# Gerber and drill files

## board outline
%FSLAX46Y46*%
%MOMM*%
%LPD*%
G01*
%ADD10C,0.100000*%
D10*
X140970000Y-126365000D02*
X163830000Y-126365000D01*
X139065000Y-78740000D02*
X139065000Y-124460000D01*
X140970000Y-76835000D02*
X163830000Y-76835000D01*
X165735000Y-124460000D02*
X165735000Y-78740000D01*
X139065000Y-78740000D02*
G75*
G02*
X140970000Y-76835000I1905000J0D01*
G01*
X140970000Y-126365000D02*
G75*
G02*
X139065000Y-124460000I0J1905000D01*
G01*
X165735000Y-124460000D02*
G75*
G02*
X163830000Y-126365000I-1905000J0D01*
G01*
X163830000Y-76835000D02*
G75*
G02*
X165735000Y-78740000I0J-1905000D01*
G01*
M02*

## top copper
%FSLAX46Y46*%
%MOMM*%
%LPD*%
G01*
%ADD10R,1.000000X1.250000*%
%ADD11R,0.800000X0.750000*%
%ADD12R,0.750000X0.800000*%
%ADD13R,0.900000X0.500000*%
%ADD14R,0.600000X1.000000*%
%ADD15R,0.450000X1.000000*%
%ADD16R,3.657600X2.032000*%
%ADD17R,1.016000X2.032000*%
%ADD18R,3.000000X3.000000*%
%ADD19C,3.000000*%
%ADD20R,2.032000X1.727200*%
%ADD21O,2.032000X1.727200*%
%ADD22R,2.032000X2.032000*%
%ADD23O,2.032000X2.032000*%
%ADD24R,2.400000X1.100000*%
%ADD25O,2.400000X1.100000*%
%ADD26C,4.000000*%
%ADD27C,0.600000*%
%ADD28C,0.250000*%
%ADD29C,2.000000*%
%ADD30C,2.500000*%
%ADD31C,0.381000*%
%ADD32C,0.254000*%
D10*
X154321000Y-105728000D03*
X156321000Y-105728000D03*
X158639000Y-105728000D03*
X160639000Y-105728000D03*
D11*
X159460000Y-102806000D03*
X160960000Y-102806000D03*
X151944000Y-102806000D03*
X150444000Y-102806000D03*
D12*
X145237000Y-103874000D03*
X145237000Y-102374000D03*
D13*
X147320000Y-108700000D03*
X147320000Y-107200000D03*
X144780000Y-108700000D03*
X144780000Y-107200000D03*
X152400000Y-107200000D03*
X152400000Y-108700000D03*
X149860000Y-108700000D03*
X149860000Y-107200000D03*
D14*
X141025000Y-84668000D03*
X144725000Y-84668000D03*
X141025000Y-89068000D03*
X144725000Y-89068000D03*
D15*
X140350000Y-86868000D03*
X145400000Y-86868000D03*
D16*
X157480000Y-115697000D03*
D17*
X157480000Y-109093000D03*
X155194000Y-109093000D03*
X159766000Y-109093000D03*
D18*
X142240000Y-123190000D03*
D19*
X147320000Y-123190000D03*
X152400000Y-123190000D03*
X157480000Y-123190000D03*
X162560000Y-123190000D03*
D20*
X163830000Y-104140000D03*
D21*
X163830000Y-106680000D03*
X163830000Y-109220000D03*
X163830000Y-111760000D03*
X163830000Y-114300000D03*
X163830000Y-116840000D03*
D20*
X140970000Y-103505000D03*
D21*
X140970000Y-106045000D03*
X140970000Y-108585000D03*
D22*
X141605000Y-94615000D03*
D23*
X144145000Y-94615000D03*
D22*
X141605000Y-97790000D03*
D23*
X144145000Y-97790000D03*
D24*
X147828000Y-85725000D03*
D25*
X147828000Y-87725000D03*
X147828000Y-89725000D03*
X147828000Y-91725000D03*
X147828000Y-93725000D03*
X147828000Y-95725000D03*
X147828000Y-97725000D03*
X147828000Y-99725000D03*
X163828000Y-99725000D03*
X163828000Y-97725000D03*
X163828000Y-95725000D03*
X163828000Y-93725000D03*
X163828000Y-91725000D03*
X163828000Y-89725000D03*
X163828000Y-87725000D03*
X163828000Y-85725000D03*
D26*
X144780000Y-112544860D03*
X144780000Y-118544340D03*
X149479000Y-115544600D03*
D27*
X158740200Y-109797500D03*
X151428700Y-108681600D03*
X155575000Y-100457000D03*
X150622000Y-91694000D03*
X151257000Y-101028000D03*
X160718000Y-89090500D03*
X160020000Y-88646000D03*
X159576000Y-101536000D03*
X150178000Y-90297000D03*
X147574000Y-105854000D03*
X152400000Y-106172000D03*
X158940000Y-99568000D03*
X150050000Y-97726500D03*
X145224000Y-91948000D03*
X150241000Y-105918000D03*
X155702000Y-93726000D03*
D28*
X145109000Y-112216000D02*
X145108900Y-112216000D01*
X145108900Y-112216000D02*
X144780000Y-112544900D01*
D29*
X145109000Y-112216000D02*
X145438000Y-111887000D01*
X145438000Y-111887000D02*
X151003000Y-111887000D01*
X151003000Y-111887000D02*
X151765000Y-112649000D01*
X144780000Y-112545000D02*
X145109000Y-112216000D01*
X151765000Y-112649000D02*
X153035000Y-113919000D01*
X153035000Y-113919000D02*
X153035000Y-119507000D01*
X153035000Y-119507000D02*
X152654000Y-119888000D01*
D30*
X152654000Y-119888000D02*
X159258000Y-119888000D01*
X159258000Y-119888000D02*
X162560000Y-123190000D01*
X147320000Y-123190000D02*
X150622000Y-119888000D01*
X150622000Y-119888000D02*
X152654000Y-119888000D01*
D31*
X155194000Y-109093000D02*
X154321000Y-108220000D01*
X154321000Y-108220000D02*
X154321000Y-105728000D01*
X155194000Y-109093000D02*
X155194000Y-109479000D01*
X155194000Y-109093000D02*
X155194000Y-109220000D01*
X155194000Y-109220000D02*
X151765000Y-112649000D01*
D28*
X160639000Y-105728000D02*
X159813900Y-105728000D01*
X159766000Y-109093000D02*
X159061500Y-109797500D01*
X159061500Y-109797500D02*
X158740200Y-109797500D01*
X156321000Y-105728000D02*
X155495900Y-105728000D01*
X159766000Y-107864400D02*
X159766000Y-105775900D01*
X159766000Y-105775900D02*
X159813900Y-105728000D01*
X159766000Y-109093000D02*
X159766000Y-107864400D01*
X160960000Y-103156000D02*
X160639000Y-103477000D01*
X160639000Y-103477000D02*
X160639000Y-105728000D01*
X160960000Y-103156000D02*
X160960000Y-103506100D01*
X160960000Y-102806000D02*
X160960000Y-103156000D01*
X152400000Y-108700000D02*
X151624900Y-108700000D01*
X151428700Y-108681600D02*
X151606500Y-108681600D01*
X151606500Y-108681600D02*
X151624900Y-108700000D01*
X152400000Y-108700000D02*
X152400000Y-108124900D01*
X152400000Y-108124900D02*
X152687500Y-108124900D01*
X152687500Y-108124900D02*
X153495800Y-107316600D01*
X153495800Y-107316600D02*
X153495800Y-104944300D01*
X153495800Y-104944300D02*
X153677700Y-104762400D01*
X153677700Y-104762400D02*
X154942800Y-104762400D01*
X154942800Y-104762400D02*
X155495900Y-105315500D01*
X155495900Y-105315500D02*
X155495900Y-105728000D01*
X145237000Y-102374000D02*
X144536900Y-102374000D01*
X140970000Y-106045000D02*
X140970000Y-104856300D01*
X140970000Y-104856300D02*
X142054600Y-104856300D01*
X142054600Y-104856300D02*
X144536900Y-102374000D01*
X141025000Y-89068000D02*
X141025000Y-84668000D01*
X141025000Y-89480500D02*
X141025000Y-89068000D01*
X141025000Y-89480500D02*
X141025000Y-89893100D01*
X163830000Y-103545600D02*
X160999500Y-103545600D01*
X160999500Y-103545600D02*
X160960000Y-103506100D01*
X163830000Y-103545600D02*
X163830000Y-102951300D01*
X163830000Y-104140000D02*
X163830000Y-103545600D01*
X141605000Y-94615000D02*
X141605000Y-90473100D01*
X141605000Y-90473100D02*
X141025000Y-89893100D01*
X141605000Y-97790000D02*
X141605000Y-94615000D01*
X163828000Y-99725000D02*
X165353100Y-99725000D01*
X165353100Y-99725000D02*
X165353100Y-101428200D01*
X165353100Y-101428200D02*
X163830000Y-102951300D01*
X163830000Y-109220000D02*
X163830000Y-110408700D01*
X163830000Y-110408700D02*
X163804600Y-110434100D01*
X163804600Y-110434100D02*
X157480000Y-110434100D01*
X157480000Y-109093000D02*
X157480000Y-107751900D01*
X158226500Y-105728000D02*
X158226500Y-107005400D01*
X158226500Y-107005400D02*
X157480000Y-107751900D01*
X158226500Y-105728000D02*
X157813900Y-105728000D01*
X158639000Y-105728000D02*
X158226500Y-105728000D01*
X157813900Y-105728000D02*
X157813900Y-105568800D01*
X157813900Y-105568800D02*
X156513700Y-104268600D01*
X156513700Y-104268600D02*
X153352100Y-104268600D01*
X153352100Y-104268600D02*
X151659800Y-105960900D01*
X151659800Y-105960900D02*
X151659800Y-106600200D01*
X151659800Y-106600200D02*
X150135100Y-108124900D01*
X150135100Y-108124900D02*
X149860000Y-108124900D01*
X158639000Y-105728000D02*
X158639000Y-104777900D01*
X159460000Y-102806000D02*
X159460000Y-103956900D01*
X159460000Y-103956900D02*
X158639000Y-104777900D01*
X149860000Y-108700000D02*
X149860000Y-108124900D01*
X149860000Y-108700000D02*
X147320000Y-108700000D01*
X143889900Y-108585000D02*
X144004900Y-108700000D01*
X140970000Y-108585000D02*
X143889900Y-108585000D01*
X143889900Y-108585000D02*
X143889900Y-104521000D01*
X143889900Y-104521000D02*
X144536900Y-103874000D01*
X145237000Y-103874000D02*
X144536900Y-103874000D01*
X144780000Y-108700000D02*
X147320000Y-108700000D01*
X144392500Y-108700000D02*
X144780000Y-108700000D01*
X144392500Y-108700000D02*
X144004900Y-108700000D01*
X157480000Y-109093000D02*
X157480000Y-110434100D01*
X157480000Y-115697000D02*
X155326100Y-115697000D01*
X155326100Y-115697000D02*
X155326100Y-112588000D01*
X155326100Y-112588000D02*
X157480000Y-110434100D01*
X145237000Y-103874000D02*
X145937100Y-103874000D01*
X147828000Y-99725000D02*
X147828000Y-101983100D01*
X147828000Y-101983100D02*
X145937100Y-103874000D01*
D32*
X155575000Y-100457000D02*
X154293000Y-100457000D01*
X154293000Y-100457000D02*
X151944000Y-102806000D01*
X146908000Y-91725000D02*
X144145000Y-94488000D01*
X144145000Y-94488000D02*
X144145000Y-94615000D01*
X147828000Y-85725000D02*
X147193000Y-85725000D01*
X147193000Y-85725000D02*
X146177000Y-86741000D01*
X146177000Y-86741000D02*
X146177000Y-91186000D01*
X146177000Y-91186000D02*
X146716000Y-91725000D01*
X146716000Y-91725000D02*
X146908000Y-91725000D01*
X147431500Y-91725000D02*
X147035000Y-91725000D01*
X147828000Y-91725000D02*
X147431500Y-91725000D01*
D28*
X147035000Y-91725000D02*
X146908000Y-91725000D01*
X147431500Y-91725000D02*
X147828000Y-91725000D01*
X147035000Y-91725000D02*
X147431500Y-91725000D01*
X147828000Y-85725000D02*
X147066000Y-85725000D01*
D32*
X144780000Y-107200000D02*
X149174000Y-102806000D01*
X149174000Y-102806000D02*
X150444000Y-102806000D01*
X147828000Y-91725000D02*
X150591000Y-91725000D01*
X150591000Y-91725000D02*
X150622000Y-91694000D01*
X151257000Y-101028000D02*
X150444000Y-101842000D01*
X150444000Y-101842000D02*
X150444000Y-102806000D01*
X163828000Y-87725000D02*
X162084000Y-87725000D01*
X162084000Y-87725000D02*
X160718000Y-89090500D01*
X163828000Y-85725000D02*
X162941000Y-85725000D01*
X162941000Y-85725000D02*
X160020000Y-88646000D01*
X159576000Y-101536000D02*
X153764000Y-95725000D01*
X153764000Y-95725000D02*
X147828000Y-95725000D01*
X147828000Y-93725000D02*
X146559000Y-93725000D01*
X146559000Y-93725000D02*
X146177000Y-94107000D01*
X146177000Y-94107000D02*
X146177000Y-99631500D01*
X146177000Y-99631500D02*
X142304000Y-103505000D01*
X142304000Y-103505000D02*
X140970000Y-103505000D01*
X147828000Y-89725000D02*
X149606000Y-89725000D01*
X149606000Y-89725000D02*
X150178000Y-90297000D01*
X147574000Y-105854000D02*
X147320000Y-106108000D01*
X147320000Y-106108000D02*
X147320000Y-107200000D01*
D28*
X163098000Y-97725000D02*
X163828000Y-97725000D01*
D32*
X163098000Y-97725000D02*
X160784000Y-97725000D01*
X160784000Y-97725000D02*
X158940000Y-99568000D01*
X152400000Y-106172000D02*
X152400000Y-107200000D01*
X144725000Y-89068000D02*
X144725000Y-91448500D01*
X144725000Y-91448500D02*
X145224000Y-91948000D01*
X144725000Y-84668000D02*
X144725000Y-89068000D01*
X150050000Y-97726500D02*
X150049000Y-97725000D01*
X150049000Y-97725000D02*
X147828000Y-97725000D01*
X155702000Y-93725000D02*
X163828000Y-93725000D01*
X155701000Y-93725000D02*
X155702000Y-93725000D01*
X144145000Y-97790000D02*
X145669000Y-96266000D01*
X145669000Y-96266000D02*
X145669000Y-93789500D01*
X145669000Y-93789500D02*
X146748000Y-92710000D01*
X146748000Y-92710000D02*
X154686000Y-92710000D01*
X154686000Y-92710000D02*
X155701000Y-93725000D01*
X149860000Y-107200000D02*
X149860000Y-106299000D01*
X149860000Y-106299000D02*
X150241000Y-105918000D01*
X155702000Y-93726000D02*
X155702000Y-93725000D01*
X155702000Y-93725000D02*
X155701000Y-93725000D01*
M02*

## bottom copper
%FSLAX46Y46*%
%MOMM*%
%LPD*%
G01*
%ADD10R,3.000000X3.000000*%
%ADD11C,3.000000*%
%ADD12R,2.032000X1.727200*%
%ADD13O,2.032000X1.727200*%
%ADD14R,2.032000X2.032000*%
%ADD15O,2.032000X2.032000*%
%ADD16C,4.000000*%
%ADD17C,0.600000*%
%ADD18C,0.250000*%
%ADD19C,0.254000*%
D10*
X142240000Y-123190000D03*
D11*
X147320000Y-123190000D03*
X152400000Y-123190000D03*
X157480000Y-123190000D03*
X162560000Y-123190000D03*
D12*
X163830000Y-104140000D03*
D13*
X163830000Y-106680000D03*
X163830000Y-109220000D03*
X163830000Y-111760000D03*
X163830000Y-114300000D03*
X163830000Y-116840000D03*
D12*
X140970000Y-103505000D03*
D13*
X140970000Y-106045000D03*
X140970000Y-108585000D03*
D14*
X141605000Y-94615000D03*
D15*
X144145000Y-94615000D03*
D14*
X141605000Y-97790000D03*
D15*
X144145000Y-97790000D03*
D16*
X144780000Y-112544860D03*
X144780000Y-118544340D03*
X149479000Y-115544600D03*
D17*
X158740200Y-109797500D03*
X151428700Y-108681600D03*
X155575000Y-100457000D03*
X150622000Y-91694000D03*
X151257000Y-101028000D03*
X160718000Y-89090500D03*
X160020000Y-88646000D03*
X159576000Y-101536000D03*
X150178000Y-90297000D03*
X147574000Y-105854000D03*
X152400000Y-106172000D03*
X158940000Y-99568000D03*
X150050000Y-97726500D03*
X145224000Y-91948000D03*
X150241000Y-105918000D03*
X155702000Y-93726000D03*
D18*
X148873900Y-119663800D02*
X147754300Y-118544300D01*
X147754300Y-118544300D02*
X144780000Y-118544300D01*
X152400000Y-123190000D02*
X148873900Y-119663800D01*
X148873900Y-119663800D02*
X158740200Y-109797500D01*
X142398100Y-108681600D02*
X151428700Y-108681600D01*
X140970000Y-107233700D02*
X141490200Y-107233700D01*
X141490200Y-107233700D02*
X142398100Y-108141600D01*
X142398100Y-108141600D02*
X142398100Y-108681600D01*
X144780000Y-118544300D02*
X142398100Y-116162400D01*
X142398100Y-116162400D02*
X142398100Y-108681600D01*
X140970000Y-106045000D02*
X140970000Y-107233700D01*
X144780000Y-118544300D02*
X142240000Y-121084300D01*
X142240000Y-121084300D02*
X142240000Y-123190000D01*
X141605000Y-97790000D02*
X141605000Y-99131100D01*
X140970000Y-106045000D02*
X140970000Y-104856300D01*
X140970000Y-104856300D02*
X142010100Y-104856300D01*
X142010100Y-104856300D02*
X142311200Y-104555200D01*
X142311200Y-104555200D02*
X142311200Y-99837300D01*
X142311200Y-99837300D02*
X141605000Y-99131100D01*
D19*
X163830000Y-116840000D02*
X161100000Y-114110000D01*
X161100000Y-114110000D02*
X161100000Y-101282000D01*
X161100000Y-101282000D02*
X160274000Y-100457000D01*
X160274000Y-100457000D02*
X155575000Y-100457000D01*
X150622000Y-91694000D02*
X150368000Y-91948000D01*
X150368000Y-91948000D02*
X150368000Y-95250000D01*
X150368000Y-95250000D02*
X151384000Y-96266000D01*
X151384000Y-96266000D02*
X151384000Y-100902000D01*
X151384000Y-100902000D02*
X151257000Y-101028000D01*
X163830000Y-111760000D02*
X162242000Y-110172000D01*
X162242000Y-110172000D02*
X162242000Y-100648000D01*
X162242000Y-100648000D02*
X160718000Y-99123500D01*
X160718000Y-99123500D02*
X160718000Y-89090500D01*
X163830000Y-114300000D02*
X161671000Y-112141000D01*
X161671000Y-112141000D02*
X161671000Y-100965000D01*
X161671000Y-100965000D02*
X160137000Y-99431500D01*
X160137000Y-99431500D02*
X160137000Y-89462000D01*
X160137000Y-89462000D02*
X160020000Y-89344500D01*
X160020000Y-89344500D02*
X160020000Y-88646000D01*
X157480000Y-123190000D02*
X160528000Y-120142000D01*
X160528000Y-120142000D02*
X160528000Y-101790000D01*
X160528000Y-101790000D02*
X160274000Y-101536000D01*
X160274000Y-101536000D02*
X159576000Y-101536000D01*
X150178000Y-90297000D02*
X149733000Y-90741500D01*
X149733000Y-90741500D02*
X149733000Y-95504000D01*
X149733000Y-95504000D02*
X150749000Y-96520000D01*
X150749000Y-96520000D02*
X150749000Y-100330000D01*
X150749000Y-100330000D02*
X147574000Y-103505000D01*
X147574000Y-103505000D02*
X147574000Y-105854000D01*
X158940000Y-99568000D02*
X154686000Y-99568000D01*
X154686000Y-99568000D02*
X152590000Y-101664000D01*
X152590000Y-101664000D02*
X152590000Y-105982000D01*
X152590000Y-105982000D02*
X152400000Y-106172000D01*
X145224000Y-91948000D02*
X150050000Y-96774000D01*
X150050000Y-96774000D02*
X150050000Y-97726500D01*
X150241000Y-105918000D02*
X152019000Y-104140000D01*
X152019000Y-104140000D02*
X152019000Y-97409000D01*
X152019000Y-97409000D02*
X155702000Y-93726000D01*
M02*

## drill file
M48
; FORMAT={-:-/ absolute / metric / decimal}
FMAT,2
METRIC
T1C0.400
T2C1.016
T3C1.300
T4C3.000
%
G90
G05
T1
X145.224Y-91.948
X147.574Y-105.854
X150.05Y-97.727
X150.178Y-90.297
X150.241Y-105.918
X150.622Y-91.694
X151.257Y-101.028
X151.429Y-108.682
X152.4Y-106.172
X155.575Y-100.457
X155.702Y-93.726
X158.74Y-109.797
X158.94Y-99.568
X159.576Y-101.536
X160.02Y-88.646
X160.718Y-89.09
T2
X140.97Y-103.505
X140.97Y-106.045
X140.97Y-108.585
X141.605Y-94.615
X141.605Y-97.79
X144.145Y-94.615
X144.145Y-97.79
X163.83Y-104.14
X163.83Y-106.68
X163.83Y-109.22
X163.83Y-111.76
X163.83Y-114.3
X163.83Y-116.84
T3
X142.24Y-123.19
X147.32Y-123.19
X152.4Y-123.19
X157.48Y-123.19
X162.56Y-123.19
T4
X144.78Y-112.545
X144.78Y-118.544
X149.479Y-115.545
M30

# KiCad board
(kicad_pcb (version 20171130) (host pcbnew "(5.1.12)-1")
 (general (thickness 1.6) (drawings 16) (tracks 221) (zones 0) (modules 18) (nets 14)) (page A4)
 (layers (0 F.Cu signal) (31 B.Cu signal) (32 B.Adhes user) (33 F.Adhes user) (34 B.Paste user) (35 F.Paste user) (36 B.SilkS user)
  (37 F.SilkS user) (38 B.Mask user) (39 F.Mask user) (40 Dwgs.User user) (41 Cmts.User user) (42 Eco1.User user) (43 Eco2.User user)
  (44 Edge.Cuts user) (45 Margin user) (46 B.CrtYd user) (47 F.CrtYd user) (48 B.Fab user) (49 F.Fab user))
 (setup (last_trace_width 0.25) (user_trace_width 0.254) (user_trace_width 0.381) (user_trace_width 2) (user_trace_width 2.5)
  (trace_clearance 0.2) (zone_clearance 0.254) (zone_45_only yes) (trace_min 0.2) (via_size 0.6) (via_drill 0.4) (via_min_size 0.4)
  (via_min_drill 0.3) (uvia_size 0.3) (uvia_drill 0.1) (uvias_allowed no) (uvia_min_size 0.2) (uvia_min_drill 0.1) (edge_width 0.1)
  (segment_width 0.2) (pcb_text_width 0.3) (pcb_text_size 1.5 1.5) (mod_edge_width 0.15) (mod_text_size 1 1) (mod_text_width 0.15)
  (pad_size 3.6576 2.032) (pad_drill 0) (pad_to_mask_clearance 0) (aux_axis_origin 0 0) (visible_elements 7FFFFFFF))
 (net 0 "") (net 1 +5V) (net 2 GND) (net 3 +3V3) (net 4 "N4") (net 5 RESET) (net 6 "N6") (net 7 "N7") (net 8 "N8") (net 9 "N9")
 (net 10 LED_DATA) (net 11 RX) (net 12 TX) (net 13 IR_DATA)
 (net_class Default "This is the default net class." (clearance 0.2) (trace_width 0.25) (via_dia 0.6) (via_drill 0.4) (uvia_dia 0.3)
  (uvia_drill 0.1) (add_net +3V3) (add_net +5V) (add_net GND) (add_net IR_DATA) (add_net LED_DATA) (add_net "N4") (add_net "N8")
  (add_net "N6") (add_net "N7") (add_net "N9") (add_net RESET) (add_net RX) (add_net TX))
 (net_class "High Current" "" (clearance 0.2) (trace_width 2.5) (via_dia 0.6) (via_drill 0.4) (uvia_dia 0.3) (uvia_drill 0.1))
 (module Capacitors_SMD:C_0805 (layer F.Cu) (at 155.321 105.728)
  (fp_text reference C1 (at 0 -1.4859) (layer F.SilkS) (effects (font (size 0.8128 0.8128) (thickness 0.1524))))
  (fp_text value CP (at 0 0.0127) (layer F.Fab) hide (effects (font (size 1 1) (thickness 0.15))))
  (pad 1 smd rect (at -1 0) (size 1 1.25) (layers F.Cu F.Paste F.Mask) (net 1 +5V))
  (pad 2 smd rect (at 1 0) (size 1 1.25) (layers F.Cu F.Paste F.Mask) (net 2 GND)))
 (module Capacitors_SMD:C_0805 (layer F.Cu) (at 159.639 105.728)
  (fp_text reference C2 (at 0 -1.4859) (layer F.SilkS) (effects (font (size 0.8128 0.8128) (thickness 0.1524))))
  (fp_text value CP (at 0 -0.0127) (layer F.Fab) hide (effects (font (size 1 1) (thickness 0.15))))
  (pad 1 smd rect (at -1 0) (size 1 1.25) (layers F.Cu F.Paste F.Mask) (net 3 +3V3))
  (pad 2 smd rect (at 1 0) (size 1 1.25) (layers F.Cu F.Paste F.Mask) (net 2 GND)))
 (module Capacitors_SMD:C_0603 (layer F.Cu) (at 160.21 102.806)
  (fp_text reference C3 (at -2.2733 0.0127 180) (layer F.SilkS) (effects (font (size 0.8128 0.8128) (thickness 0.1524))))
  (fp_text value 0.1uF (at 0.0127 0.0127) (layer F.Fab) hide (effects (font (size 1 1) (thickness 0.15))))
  (pad 1 smd rect (at -0.75 0) (size 0.8 0.75) (layers F.Cu F.Paste F.Mask) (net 3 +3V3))
  (pad 2 smd rect (at 0.75 0) (size 0.8 0.75) (layers F.Cu F.Paste F.Mask) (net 2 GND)))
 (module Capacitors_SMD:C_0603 (layer F.Cu) (at 151.194 102.806 180)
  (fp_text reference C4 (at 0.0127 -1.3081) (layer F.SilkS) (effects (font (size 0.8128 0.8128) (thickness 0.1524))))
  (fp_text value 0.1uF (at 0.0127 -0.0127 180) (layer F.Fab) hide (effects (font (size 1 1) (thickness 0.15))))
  (pad 1 smd rect (at -0.75 0 180) (size 0.8 0.75) (layers F.Cu F.Paste F.Mask) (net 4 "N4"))
  (pad 2 smd rect (at 0.75 0 180) (size 0.8 0.75) (layers F.Cu F.Paste F.Mask) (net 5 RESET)))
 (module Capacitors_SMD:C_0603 (layer F.Cu) (at 145.237 103.124 90)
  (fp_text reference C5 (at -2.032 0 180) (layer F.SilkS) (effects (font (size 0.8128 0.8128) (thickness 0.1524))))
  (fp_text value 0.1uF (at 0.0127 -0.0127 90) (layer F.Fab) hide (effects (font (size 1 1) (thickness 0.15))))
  (pad 1 smd rect (at -0.75 0 90) (size 0.8 0.75) (layers F.Cu F.Paste F.Mask) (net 3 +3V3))
  (pad 2 smd rect (at 0.75 0 90) (size 0.8 0.75) (layers F.Cu F.Paste F.Mask) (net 2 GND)))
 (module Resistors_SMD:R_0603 (layer F.Cu) (at 147.32 107.95 90)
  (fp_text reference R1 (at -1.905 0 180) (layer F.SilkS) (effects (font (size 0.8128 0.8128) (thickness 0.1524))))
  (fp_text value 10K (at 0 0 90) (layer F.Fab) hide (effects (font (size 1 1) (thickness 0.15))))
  (pad 1 smd rect (at -0.75 0 90) (size 0.5 0.9) (layers F.Cu F.Paste F.Mask) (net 3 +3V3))
  (pad 2 smd rect (at 0.75 0 90) (size 0.5 0.9) (layers F.Cu F.Paste F.Mask) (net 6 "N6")))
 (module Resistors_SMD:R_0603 (layer F.Cu) (at 144.78 107.95 90)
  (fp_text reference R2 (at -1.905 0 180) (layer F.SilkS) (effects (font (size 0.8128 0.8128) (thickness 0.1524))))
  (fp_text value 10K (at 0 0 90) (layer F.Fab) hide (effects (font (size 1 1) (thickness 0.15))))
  (pad 1 smd rect (at -0.75 0 90) (size 0.5 0.9) (layers F.Cu F.Paste F.Mask) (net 3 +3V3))
  (pad 2 smd rect (at 0.75 0 90) (size 0.5 0.9) (layers F.Cu F.Paste F.Mask) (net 5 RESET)))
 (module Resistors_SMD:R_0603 (layer F.Cu) (at 152.4 107.95 270)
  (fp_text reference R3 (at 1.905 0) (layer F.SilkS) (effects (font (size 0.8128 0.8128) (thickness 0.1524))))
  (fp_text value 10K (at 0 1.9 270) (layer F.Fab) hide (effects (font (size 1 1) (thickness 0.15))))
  (pad 1 smd rect (at -0.75 0 270) (size 0.5 0.9) (layers F.Cu F.Paste F.Mask) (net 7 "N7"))
  (pad 2 smd rect (at 0.75 0 270) (size 0.5 0.9) (layers F.Cu F.Paste F.Mask) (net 2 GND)))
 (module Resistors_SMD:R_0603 (layer F.Cu) (at 149.86 107.95 90)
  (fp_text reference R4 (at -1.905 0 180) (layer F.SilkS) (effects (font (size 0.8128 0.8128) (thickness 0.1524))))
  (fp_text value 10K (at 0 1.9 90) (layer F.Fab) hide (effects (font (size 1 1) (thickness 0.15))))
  (pad 1 smd rect (at -0.75 0 90) (size 0.5 0.9) (layers F.Cu F.Paste F.Mask) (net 3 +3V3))
  (pad 2 smd rect (at 0.75 0 90) (size 0.5 0.9) (layers F.Cu F.Paste F.Mask) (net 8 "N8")))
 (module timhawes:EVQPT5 (layer F.Cu) (at 142.875 86.868)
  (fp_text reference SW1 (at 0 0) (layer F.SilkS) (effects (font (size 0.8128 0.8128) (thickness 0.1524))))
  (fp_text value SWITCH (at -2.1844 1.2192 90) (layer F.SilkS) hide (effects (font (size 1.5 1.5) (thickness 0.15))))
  (pad 1 smd rect (at -1.85 -2.2) (size 0.6 1) (layers F.Cu F.Paste F.Mask) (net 2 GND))
  (pad 2 smd rect (at 1.85 -2.2) (size 0.6 1) (layers F.Cu F.Paste F.Mask) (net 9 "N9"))
  (pad 1 smd rect (at -1.85 2.2) (size 0.6 1) (layers F.Cu F.Paste F.Mask) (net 2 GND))
  (pad 2 smd rect (at 1.85 2.2) (size 0.6 1) (layers F.Cu F.Paste F.Mask) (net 9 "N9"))
  (pad "" smd rect (at -2.525 0) (size 0.45 1) (layers F.Cu F.Paste F.Mask))
  (pad "" smd rect (at 2.525 0) (size 0.45 1) (layers F.Cu F.Paste F.Mask)))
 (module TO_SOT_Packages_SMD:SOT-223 (layer F.Cu) (at 157.48 112.395 180)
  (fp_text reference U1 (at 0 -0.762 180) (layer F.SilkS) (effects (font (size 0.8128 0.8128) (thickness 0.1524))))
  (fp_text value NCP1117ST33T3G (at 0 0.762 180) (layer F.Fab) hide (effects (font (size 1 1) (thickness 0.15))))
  (pad 4 smd rect (at 0 -3.302 180) (size 3.6576 2.032) (layers F.Cu F.Paste F.Mask) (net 3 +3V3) (zone_connect 2))
  (pad 2 smd rect (at 0 3.302 180) (size 1.016 2.032) (layers F.Cu F.Paste F.Mask) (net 3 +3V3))
  (pad 3 smd rect (at 2.286 3.302 180) (size 1.016 2.032) (layers F.Cu F.Paste F.Mask) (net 1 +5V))
  (pad 1 smd rect (at -2.286 3.302 180) (size 1.016 2.032) (layers F.Cu F.Paste F.Mask) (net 2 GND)))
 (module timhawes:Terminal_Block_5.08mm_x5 (layer F.Cu) (at 152.4 123.19)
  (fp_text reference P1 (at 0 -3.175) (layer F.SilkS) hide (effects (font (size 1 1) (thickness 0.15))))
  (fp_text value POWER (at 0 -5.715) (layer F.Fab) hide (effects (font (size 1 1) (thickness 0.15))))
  (pad 1 thru_hole rect (at -10.16 0) (size 3 3) (drill 1.3) (layers *.Cu *.Mask F.SilkS) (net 2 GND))
  (pad 2 thru_hole circle (at -5.08 0) (size 3 3) (drill 1.3) (layers *.Cu *.Mask F.SilkS) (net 1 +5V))
  (pad 3 thru_hole circle (at 0 0) (size 3 3) (drill 1.3) (layers *.Cu *.Mask F.SilkS) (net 2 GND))
  (pad 4 thru_hole circle (at 5.08 0) (size 3 3) (drill 1.3) (layers *.Cu *.Mask F.SilkS) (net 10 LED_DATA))
  (pad 5 thru_hole circle (at 10.16 0) (size 3 3) (drill 1.3) (layers *.Cu *.Mask F.SilkS) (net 1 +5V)))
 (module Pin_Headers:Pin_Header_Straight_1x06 (layer F.Cu) (at 163.83 104.14)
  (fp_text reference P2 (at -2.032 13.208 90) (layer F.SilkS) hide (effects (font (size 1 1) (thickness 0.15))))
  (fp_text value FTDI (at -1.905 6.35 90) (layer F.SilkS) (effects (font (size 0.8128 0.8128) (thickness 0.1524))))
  (pad 1 thru_hole rect (at 0 0) (size 2.032 1.7272) (drill 1.016) (layers *.Cu *.Mask F.SilkS) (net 2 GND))
  (pad 2 thru_hole oval (at 0 2.54) (size 2.032 1.7272) (drill 1.016) (layers *.Cu *.Mask F.SilkS))
  (pad 3 thru_hole oval (at 0 5.08) (size 2.032 1.7272) (drill 1.016) (layers *.Cu *.Mask F.SilkS) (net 3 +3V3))
  (pad 4 thru_hole oval (at 0 7.62) (size 2.032 1.7272) (drill 1.016) (layers *.Cu *.Mask F.SilkS) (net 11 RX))
  (pad 5 thru_hole oval (at 0 10.16) (size 2.032 1.7272) (drill 1.016) (layers *.Cu *.Mask F.SilkS) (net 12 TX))
  (pad 6 thru_hole oval (at 0 12.7) (size 2.032 1.7272) (drill 1.016) (layers *.Cu *.Mask F.SilkS) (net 4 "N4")))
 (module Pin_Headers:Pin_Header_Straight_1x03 (layer F.Cu) (at 140.97 103.505)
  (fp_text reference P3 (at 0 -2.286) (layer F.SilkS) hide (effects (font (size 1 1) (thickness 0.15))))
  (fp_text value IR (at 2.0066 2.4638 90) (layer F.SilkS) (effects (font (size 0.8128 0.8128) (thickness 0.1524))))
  (pad 1 thru_hole rect (at 0 0) (size 2.032 1.7272) (drill 1.016) (layers *.Cu *.Mask F.SilkS) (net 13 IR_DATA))
  (pad 2 thru_hole oval (at 0 2.54) (size 2.032 1.7272) (drill 1.016) (layers *.Cu *.Mask F.SilkS) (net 2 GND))
  (pad 3 thru_hole oval (at 0 5.08) (size 2.032 1.7272) (drill 1.016) (layers *.Cu *.Mask F.SilkS) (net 3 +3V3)))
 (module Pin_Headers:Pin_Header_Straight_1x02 (layer F.Cu) (at 141.605 94.615 90)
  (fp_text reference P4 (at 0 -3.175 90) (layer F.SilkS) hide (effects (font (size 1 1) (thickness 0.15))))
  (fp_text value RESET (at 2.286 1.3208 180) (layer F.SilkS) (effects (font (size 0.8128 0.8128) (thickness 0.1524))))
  (pad 1 thru_hole rect (at 0 0 90) (size 2.032 2.032) (drill 1.016) (layers *.Cu *.Mask F.SilkS) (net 2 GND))
  (pad 2 thru_hole oval (at 0 2.54 90) (size 2.032 2.032) (drill 1.016) (layers *.Cu *.Mask F.SilkS) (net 5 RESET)))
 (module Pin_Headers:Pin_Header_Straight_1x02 (layer F.Cu) (at 141.605 97.79 90)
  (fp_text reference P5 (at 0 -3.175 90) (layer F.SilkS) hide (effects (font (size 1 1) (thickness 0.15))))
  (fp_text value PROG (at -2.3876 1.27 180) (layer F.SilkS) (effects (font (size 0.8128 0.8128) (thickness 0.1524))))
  (pad 1 thru_hole rect (at 0 0 90) (size 2.032 2.032) (drill 1.016) (layers *.Cu *.Mask F.SilkS) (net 2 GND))
  (pad 2 thru_hole oval (at 0 2.54 90) (size 2.032 2.032) (drill 1.016) (layers *.Cu *.Mask F.SilkS) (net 8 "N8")))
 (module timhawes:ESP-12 (layer F.Cu) (at 147.828 85.725)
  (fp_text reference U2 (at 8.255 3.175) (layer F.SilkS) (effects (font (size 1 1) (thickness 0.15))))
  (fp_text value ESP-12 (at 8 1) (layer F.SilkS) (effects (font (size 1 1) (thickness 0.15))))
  (pad 1 smd rect (at 0 0) (size 2.4 1.1) (layers F.Cu F.Paste F.Mask) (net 5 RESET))
  (pad 2 smd oval (at 0 2) (size 2.4 1.1) (layers F.Cu F.Paste F.Mask))
  (pad 3 smd oval (at 0 4) (size 2.4 1.1) (layers F.Cu F.Paste F.Mask) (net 6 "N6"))
  (pad 4 smd oval (at 0 6) (size 2.4 1.1) (layers F.Cu F.Paste F.Mask) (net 5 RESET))
  (pad 5 smd oval (at 0 8) (size 2.4 1.1) (layers F.Cu F.Paste F.Mask) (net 13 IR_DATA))
  (pad 6 smd oval (at 0 10) (size 2.4 1.1) (layers F.Cu F.Paste F.Mask) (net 10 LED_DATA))
  (pad 7 smd oval (at 0 12) (size 2.4 1.1) (layers F.Cu F.Paste F.Mask) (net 9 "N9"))
  (pad 8 smd oval (at 0 14) (size 2.4 1.1) (layers F.Cu F.Paste F.Mask) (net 3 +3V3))
  (pad 9 smd oval (at 16 14) (size 2.4 1.1) (layers F.Cu F.Paste F.Mask) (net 2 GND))
  (pad 10 smd oval (at 16 12) (size 2.4 1.1) (layers F.Cu F.Paste F.Mask) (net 7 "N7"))
  (pad 11 smd oval (at 16 10) (size 2.4 1.1) (layers F.Cu F.Paste F.Mask))
  (pad 12 smd oval (at 16 8) (size 2.4 1.1) (layers F.Cu F.Paste F.Mask) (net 8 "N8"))
  (pad 13 smd oval (at 16 6) (size 2.4 1.1) (layers F.Cu F.Paste F.Mask))
  (pad 14 smd oval (at 16 4) (size 2.4 1.1) (layers F.Cu F.Paste F.Mask))
  (pad 15 smd oval (at 16 2) (size 2.4 1.1) (layers F.Cu F.Paste F.Mask) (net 11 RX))
  (pad 16 smd oval (at 16 0) (size 2.4 1.1) (layers F.Cu F.Paste F.Mask) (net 12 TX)))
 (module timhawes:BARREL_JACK (layer F.Cu) (at 144.78 118.745 90)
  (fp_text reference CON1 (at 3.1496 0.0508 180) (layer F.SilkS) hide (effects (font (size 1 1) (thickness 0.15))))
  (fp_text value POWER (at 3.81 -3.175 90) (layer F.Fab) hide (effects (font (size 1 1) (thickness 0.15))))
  (pad 1 thru_hole circle (at 6.20014 0 90) (size 4 4) (drill 3) (layers *.Cu *.Mask F.SilkS) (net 1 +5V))
  (pad 2 thru_hole circle (at 0.20066 0 90) (size 4 4) (drill 3) (layers *.Cu *.Mask F.SilkS) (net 2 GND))
  (pad 3 thru_hole circle (at 3.2004 4.699 90) (size 4 4) (drill 3) (layers *.Cu *.Mask F.SilkS)))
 (gr_line (start 140.97 126.365) (end 163.83 126.365) (angle 90) (layer Edge.Cuts) (width 0.1))
 (gr_line (start 139.065 78.74) (end 139.065 124.46) (angle 90) (layer Edge.Cuts) (width 0.1))
 (gr_line (start 140.97 76.835) (end 163.83 76.835) (angle 90) (layer Edge.Cuts) (width 0.1))
 (gr_line (start 165.735 124.46) (end 165.735 78.74) (angle 90) (layer Edge.Cuts) (width 0.1))
 (gr_arc (start 140.97 78.74) (end 139.065 78.74) (angle 90) (layer Edge.Cuts) (width 0.1))
 (gr_arc (start 140.97 124.46) (end 140.97 126.365) (angle 90) (layer Edge.Cuts) (width 0.1))
 (gr_arc (start 163.83 124.46) (end 165.735 124.46) (angle 90) (layer Edge.Cuts) (width 0.1))
 (gr_arc (start 163.83 78.74) (end 163.83 76.835) (angle 90) (layer Edge.Cuts) (width 0.1))
 (segment (start 145.109 112.216) (end 145.1089 112.216) (width 0.25) (layer F.Cu) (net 1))
 (segment (start 145.1089 112.216) (end 144.78 112.5449) (width 0.25) (layer F.Cu) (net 1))
 (segment (start 145.109 112.216) (end 145.438 111.887) (width 2) (layer F.Cu) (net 1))
 (segment (start 145.438 111.887) (end 151.003 111.887) (width 2) (layer F.Cu) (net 1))
 (segment (start 151.003 111.887) (end 151.765 112.649) (width 2) (layer F.Cu) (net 1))
 (segment (start 144.78 112.545) (end 145.109 112.216) (width 2) (layer F.Cu) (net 1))
 (segment (start 151.765 112.649) (end 153.035 113.919) (width 2) (layer F.Cu) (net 1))
 (segment (start 153.035 113.919) (end 153.035 119.507) (width 2) (layer F.Cu) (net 1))
 (segment (start 153.035 119.507) (end 152.654 119.888) (width 2) (layer F.Cu) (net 1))
 (segment (start 152.654 119.888) (end 159.258 119.888) (width 2.5) (layer F.Cu) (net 1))
 (segment (start 159.258 119.888) (end 162.56 123.19) (width 2.5) (layer F.Cu) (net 1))
 (segment (start 147.32 123.19) (end 150.622 119.888) (width 2.5) (layer F.Cu) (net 1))
 (segment (start 150.622 119.888) (end 152.654 119.888) (width 2.5) (layer F.Cu) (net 1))
 (segment (start 155.194 109.093) (end 154.321 108.22) (width 0.381) (layer F.Cu) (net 1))
 (segment (start 154.321 108.22) (end 154.321 105.728) (width 0.381) (layer F.Cu) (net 1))
 (segment (start 155.194 109.093) (end 155.194 109.479) (width 0.381) (layer F.Cu) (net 1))
 (segment (start 155.194 109.093) (end 155.194 109.22) (width 0.381) (layer F.Cu) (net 1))
 (segment (start 155.194 109.22) (end 151.765 112.649) (width 0.381) (layer F.Cu) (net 1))
 (segment (start 160.639 105.728) (end 159.8139 105.728) (width 0.25) (layer F.Cu) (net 2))
 (segment (start 148.8739 119.6638) (end 147.7543 118.5443) (width 0.25) (layer B.Cu) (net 2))
 (segment (start 147.7543 118.5443) (end 144.78 118.5443) (width 0.25) (layer B.Cu) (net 2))
 (segment (start 152.4 123.19) (end 148.8739 119.6638) (width 0.25) (layer B.Cu) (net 2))
 (segment (start 148.8739 119.6638) (end 158.7402 109.7975) (width 0.25) (layer B.Cu) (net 2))
 (segment (start 159.766 109.093) (end 159.0615 109.7975) (width 0.25) (layer F.Cu) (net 2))
 (segment (start 159.0615 109.7975) (end 158.7402 109.7975) (width 0.25) (layer F.Cu) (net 2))
 (segment (start 156.321 105.728) (end 155.4959 105.728) (width 0.25) (layer F.Cu) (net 2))
 (segment (start 159.766 107.8644) (end 159.766 105.7759) (width 0.25) (layer F.Cu) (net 2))
 (segment (start 159.766 105.7759) (end 159.8139 105.728) (width 0.25) (layer F.Cu) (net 2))
 (segment (start 159.766 109.093) (end 159.766 107.8644) (width 0.25) (layer F.Cu) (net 2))
 (segment (start 160.96 103.156) (end 160.639 103.477) (width 0.25) (layer F.Cu) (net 2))
 (segment (start 160.639 103.477) (end 160.639 105.728) (width 0.25) (layer F.Cu) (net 2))
 (segment (start 160.96 103.156) (end 160.96 103.5061) (width 0.25) (layer F.Cu) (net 2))
 (segment (start 160.96 102.806) (end 160.96 103.156) (width 0.25) (layer F.Cu) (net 2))
 (segment (start 142.3981 108.6816) (end 151.4287 108.6816) (width 0.25) (layer B.Cu) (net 2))
 (segment (start 140.97 107.2337) (end 141.4902 107.2337) (width 0.25) (layer B.Cu) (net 2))
 (segment (start 141.4902 107.2337) (end 142.3981 108.1416) (width 0.25) (layer B.Cu) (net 2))
 (segment (start 142.3981 108.1416) (end 142.3981 108.6816) (width 0.25) (layer B.Cu) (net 2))
 (segment (start 144.78 118.5443) (end 142.3981 116.1624) (width 0.25) (layer B.Cu) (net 2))
 (segment (start 142.3981 116.1624) (end 142.3981 108.6816) (width 0.25) (layer B.Cu) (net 2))
 (segment (start 152.4 108.7) (end 151.6249 108.7) (width 0.25) (layer F.Cu) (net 2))
 (segment (start 151.4287 108.6816) (end 151.6065 108.6816) (width 0.25) (layer F.Cu) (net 2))
 (segment (start 151.6065 108.6816) (end 151.6249 108.7) (width 0.25) (layer F.Cu) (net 2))
 (segment (start 152.4 108.7) (end 152.4 108.1249) (width 0.25) (layer F.Cu) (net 2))
 (segment (start 152.4 108.1249) (end 152.6875 108.1249) (width 0.25) (layer F.Cu) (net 2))
 (segment (start 152.6875 108.1249) (end 153.4958 107.3166) (width 0.25) (layer F.Cu) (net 2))
 (segment (start 153.4958 107.3166) (end 153.4958 104.9443) (width 0.25) (layer F.Cu) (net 2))
 (segment (start 153.4958 104.9443) (end 153.6777 104.7624) (width 0.25) (layer F.Cu) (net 2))
 (segment (start 153.6777 104.7624) (end 154.9428 104.7624) (width 0.25) (layer F.Cu) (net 2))
 (segment (start 154.9428 104.7624) (end 155.4959 105.3155) (width 0.25) (layer F.Cu) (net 2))
 (segment (start 155.4959 105.3155) (end 155.4959 105.728) (width 0.25) (layer F.Cu) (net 2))
 (segment (start 145.237 102.374) (end 144.5369 102.374) (width 0.25) (layer F.Cu) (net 2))
 (segment (start 140.97 106.045) (end 140.97 104.8563) (width 0.25) (layer F.Cu) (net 2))
 (segment (start 140.97 104.8563) (end 142.0546 104.8563) (width 0.25) (layer F.Cu) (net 2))
 (segment (start 142.0546 104.8563) (end 144.5369 102.374) (width 0.25) (layer F.Cu) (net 2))
 (segment (start 141.025 89.068) (end 141.025 84.668) (width 0.25) (layer F.Cu) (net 2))
 (segment (start 141.025 89.4805) (end 141.025 89.068) (width 0.25) (layer F.Cu) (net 2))
 (segment (start 141.025 89.4805) (end 141.025 89.8931) (width 0.25) (layer F.Cu) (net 2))
 (segment (start 140.97 106.045) (end 140.97 107.2337) (width 0.25) (layer B.Cu) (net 2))
 (segment (start 144.78 118.5443) (end 142.24 121.0843) (width 0.25) (layer B.Cu) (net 2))
 (segment (start 142.24 121.0843) (end 142.24 123.19) (width 0.25) (layer B.Cu) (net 2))
 (segment (start 163.83 103.5456) (end 160.9995 103.5456) (width 0.25) (layer F.Cu) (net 2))
 (segment (start 160.9995 103.5456) (end 160.96 103.5061) (width 0.25) (layer F.Cu) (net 2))
 (segment (start 163.83 103.5456) (end 163.83 102.9513) (width 0.25) (layer F.Cu) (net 2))
 (segment (start 163.83 104.14) (end 163.83 103.5456) (width 0.25) (layer F.Cu) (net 2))
 (segment (start 141.605 97.79) (end 141.605 99.1311) (width 0.25) (layer B.Cu) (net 2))
 (segment (start 140.97 106.045) (end 140.97 104.8563) (width 0.25) (layer B.Cu) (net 2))
 (segment (start 140.97 104.8563) (end 142.0101 104.8563) (width 0.25) (layer B.Cu) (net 2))
 (segment (start 142.0101 104.8563) (end 142.3112 104.5552) (width 0.25) (layer B.Cu) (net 2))
 (segment (start 142.3112 104.5552) (end 142.3112 99.8373) (width 0.25) (layer B.Cu) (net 2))
 (segment (start 142.3112 99.8373) (end 141.605 99.1311) (width 0.25) (layer B.Cu) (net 2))
 (segment (start 141.605 94.615) (end 141.605 90.4731) (width 0.25) (layer F.Cu) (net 2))
 (segment (start 141.605 90.4731) (end 141.025 89.8931) (width 0.25) (layer F.Cu) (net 2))
 (segment (start 141.605 97.79) (end 141.605 94.615) (width 0.25) (layer F.Cu) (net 2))
 (segment (start 163.828 99.725) (end 165.3531 99.725) (width 0.25) (layer F.Cu) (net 2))
 (segment (start 165.3531 99.725) (end 165.3531 101.4282) (width 0.25) (layer F.Cu) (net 2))
 (segment (start 165.3531 101.4282) (end 163.83 102.9513) (width 0.25) (layer F.Cu) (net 2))
 (via (at 158.7402 109.7975) (size 0.6) (layers F.Cu B.Cu) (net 2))
 (via (at 151.4287 108.6816) (size 0.6) (layers F.Cu B.Cu) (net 2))
 (segment (start 163.83 109.22) (end 163.83 110.4087) (width 0.25) (layer F.Cu) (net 3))
 (segment (start 163.83 110.4087) (end 163.8046 110.4341) (width 0.25) (layer F.Cu) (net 3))
 (segment (start 163.8046 110.4341) (end 157.48 110.4341) (width 0.25) (layer F.Cu) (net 3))
 (segment (start 157.48 109.093) (end 157.48 107.7519) (width 0.25) (layer F.Cu) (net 3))
 (segment (start 158.2265 105.728) (end 158.2265 107.0054) (width 0.25) (layer F.Cu) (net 3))
 (segment (start 158.2265 107.0054) (end 157.48 107.7519) (width 0.25) (layer F.Cu) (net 3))
 (segment (start 158.2265 105.728) (end 157.8139 105.728) (width 0.25) (layer F.Cu) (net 3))
 (segment (start 158.639 105.728) (end 158.2265 105.728) (width 0.25) (layer F.Cu) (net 3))
 (segment (start 157.8139 105.728) (end 157.8139 105.5688) (width 0.25) (layer F.Cu) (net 3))
 (segment (start 157.8139 105.5688) (end 156.5137 104.2686) (width 0.25) (layer F.Cu) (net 3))
 (segment (start 156.5137 104.2686) (end 153.3521 104.2686) (width 0.25) (layer F.Cu) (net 3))
 (segment (start 153.3521 104.2686) (end 151.6598 105.9609) (width 0.25) (layer F.Cu) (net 3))
 (segment (start 151.6598 105.9609) (end 151.6598 106.6002) (width 0.25) (layer F.Cu) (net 3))
 (segment (start 151.6598 106.6002) (end 150.1351 108.1249) (width 0.25) (layer F.Cu) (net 3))
 (segment (start 150.1351 108.1249) (end 149.86 108.1249) (width 0.25) (layer F.Cu) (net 3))
 (segment (start 158.639 105.728) (end 158.639 104.7779) (width 0.25) (layer F.Cu) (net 3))
 (segment (start 159.46 102.806) (end 159.46 103.9569) (width 0.25) (layer F.Cu) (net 3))
 (segment (start 159.46 103.9569) (end 158.639 104.7779) (width 0.25) (layer F.Cu) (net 3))
 (segment (start 149.86 108.7) (end 149.86 108.1249) (width 0.25) (layer F.Cu) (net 3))
 (segment (start 149.86 108.7) (end 147.32 108.7) (width 0.25) (layer F.Cu) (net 3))
 (segment (start 143.8899 108.585) (end 144.0049 108.7) (width 0.25) (layer F.Cu) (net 3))
 (segment (start 140.97 108.585) (end 143.8899 108.585) (width 0.25) (layer F.Cu) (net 3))
 (segment (start 143.8899 108.585) (end 143.8899 104.521) (width 0.25) (layer F.Cu) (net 3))
 (segment (start 143.8899 104.521) (end 144.5369 103.874) (width 0.25) (layer F.Cu) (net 3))
 (segment (start 145.237 103.874) (end 144.5369 103.874) (width 0.25) (layer F.Cu) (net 3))
 (segment (start 144.78 108.7) (end 147.32 108.7) (width 0.25) (layer F.Cu) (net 3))
 (segment (start 144.3925 108.7) (end 144.78 108.7) (width 0.25) (layer F.Cu) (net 3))
 (segment (start 144.3925 108.7) (end 144.0049 108.7) (width 0.25) (layer F.Cu) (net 3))
 (segment (start 157.48 109.093) (end 157.48 110.4341) (width 0.25) (layer F.Cu) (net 3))
 (segment (start 157.48 115.697) (end 155.3261 115.697) (width 0.25) (layer F.Cu) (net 3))
 (segment (start 155.3261 115.697) (end 155.3261 112.588) (width 0.25) (layer F.Cu) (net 3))
 (segment (start 155.3261 112.588) (end 157.48 110.4341) (width 0.25) (layer F.Cu) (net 3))
 (segment (start 145.237 103.874) (end 145.9371 103.874) (width 0.25) (layer F.Cu) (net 3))
 (segment (start 147.828 99.725) (end 147.828 101.9831) (width 0.25) (layer F.Cu) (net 3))
 (segment (start 147.828 101.9831) (end 145.9371 103.874) (width 0.25) (layer F.Cu) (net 3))
 (segment (start 155.575 100.457) (end 154.293 100.457) (width 0.254) (layer F.Cu) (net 4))
 (segment (start 154.293 100.457) (end 151.944 102.806) (width 0.254) (layer F.Cu) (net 4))
 (segment (start 163.83 116.84) (end 161.1 114.11) (width 0.254) (layer B.Cu) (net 4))
 (segment (start 161.1 114.11) (end 161.1 101.282) (width 0.254) (layer B.Cu) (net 4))
 (segment (start 161.1 101.282) (end 160.274 100.457) (width 0.254) (layer B.Cu) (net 4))
 (segment (start 160.274 100.457) (end 155.575 100.457) (width 0.254) (layer B.Cu) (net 4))
 (via (at 155.575 100.457) (size 0.6) (layers F.Cu B.Cu) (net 4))
 (segment (start 146.908 91.725) (end 144.145 94.488) (width 0.254) (layer F.Cu) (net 5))
 (segment (start 144.145 94.488) (end 144.145 94.615) (width 0.254) (layer F.Cu) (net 5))
 (segment (start 147.828 85.725) (end 147.193 85.725) (width 0.254) (layer F.Cu) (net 5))
 (segment (start 147.193 85.725) (end 146.177 86.741) (width 0.254) (layer F.Cu) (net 5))
 (segment (start 146.177 86.741) (end 146.177 91.186) (width 0.254) (layer F.Cu) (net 5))
 (segment (start 146.177 91.186) (end 146.716 91.725) (width 0.254) (layer F.Cu) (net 5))
 (segment (start 146.716 91.725) (end 146.908 91.725) (width 0.254) (layer F.Cu) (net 5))
 (segment (start 147.4315 91.725) (end 147.035 91.725) (width 0.254) (layer F.Cu) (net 5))
 (segment (start 147.828 91.725) (end 147.4315 91.725) (width 0.254) (layer F.Cu) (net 5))
 (segment (start 147.035 91.725) (end 146.908 91.725) (width 0.25) (layer F.Cu) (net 5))
 (segment (start 147.4315 91.725) (end 147.828 91.725) (width 0.25) (layer F.Cu) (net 5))
 (segment (start 147.035 91.725) (end 147.4315 91.725) (width 0.25) (layer F.Cu) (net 5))
 (segment (start 147.828 85.725) (end 147.066 85.725) (width 0.25) (layer F.Cu) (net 5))
 (segment (start 144.78 107.2) (end 149.174 102.806) (width 0.254) (layer F.Cu) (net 5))
 (segment (start 149.174 102.806) (end 150.444 102.806) (width 0.254) (layer F.Cu) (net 5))
 (segment (start 150.622 91.694) (end 150.368 91.948) (width 0.254) (layer B.Cu) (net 5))
 (segment (start 150.368 91.948) (end 150.368 95.25) (width 0.254) (layer B.Cu) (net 5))
 (segment (start 150.368 95.25) (end 151.384 96.266) (width 0.254) (layer B.Cu) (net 5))
 (segment (start 151.384 96.266) (end 151.384 100.902) (width 0.254) (layer B.Cu) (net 5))
 (segment (start 151.384 100.902) (end 151.257 101.028) (width 0.254) (layer B.Cu) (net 5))
 (segment (start 147.828 91.725) (end 150.591 91.725) (width 0.254) (layer F.Cu) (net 5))
 (segment (start 150.591 91.725) (end 150.622 91.694) (width 0.254) (layer F.Cu) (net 5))
 (segment (start 151.257 101.028) (end 150.444 101.842) (width 0.254) (layer F.Cu) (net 5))
 (segment (start 150.444 101.842) (end 150.444 102.806) (width 0.254) (layer F.Cu) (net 5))
 (via (at 150.622 91.694) (size 0.6) (layers F.Cu B.Cu) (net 5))
 (via (at 151.257 101.028) (size 0.6) (layers F.Cu B.Cu) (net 5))
 (segment (start 163.828 87.725) (end 162.084 87.725) (width 0.254) (layer F.Cu) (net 11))
 (segment (start 162.084 87.725) (end 160.718 89.0905) (width 0.254) (layer F.Cu) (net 11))
 (segment (start 163.83 111.76) (end 162.242 110.172) (width 0.254) (layer B.Cu) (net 11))
 (segment (start 162.242 110.172) (end 162.242 100.648) (width 0.254) (layer B.Cu) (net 11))
 (segment (start 162.242 100.648) (end 160.718 99.1235) (width 0.254) (layer B.Cu) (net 11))
 (segment (start 160.718 99.1235) (end 160.718 89.0905) (width 0.254) (layer B.Cu) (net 11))
 (via (at 160.718 89.0905) (size 0.6) (layers F.Cu B.Cu) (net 11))
 (segment (start 163.83 114.3) (end 161.671 112.141) (width 0.254) (layer B.Cu) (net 12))
 (segment (start 161.671 112.141) (end 161.671 100.965) (width 0.254) (layer B.Cu) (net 12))
 (segment (start 161.671 100.965) (end 160.137 99.4315) (width 0.254) (layer B.Cu) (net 12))
 (segment (start 160.137 99.4315) (end 160.137 89.462) (width 0.254) (layer B.Cu) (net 12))
 (segment (start 160.137 89.462) (end 160.02 89.3445) (width 0.254) (layer B.Cu) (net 12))
 (segment (start 160.02 89.3445) (end 160.02 88.646) (width 0.254) (layer B.Cu) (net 12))
 (segment (start 163.828 85.725) (end 162.941 85.725) (width 0.254) (layer F.Cu) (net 12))
 (segment (start 162.941 85.725) (end 160.02 88.646) (width 0.254) (layer F.Cu) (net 12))
 (via (at 160.02 88.646) (size 0.6) (layers F.Cu B.Cu) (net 12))
 (segment (start 157.48 123.19) (end 160.528 120.142) (width 0.254) (layer B.Cu) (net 10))
 (segment (start 160.528 120.142) (end 160.528 101.79) (width 0.254) (layer B.Cu) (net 10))
 (segment (start 160.528 101.79) (end 160.274 101.536) (width 0.254) (layer B.Cu) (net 10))
 (segment (start 160.274 101.536) (end 159.576 101.536) (width 0.254) (layer B.Cu) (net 10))
 (segment (start 159.576 101.536) (end 153.764 95.725) (width 0.254) (layer F.Cu) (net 10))
 (segment (start 153.764 95.725) (end 147.828 95.725) (width 0.254) (layer F.Cu) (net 10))
 (via (at 159.576 101.536) (size 0.6) (layers F.Cu B.Cu) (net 10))
 (segment (start 147.828 93.725) (end 146.559 93.725) (width 0.254) (layer F.Cu) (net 13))
 (segment (start 146.559 93.725) (end 146.177 94.107) (width 0.254) (layer F.Cu) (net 13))
 (segment (start 146.177 94.107) (end 146.177 99.6315) (width 0.254) (layer F.Cu) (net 13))
 (segment (start 146.177 99.6315) (end 142.304 103.505) (width 0.254) (layer F.Cu) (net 13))
 (segment (start 142.304 103.505) (end 140.97 103.505) (width 0.254) (layer F.Cu) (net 13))
 (segment (start 147.828 89.725) (end 149.606 89.725) (width 0.254) (layer F.Cu) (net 6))
 (segment (start 149.606 89.725) (end 150.178 90.297) (width 0.254) (layer F.Cu) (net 6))
 (segment (start 150.178 90.297) (end 149.733 90.7415) (width 0.254) (layer B.Cu) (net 6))
 (segment (start 149.733 90.7415) (end 149.733 95.504) (width 0.254) (layer B.Cu) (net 6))
 (segment (start 149.733 95.504) (end 150.749 96.52) (width 0.254) (layer B.Cu) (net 6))
 (segment (start 150.749 96.52) (end 150.749 100.33) (width 0.254) (layer B.Cu) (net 6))
 (segment (start 150.749 100.33) (end 147.574 103.505) (width 0.254) (layer B.Cu) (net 6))
 (segment (start 147.574 103.505) (end 147.574 105.854) (width 0.254) (layer B.Cu) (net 6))
 (segment (start 147.574 105.854) (end 147.32 106.108) (width 0.254) (layer F.Cu) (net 6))
 (segment (start 147.32 106.108) (end 147.32 107.2) (width 0.254) (layer F.Cu) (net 6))
 (via (at 150.178 90.297) (size 0.6) (layers F.Cu B.Cu) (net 6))
 (via (at 147.574 105.854) (size 0.6) (layers F.Cu B.Cu) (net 6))
 (segment (start 163.098 97.725) (end 163.828 97.725) (width 0.25) (layer F.Cu) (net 7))
 (segment (start 163.098 97.725) (end 160.784 97.725) (width 0.254) (layer F.Cu) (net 7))
 (segment (start 160.784 97.725) (end 158.94 99.568) (width 0.254) (layer F.Cu) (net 7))
 (segment (start 158.94 99.568) (end 154.686 99.568) (width 0.254) (layer B.Cu) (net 7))
 (segment (start 154.686 99.568) (end 152.59 101.664) (width 0.254) (layer B.Cu) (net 7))
 (segment (start 152.59 101.664) (end 152.59 105.982) (width 0.254) (layer B.Cu) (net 7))
 (segment (start 152.59 105.982) (end 152.4 106.172) (width 0.254) (layer B.Cu) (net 7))
 (segment (start 152.4 106.172) (end 152.4 107.2) (width 0.254) (layer F.Cu) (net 7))
 (via (at 152.4 106.172) (size 0.6) (layers F.Cu B.Cu) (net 7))
 (via (at 158.94 99.568) (size 0.6) (layers F.Cu B.Cu) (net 7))
 (segment (start 144.725 89.068) (end 144.725 91.4485) (width 0.254) (layer F.Cu) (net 9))
 (segment (start 144.725 91.4485) (end 145.224 91.948) (width 0.254) (layer F.Cu) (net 9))
 (segment (start 144.725 84.668) (end 144.725 89.068) (width 0.254) (layer F.Cu) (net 9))
 (segment (start 150.05 97.7265) (end 150.049 97.725) (width 0.254) (layer F.Cu) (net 9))
 (segment (start 150.049 97.725) (end 147.828 97.725) (width 0.254) (layer F.Cu) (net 9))
 (segment (start 145.224 91.948) (end 150.05 96.774) (width 0.254) (layer B.Cu) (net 9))
 (segment (start 150.05 96.774) (end 150.05 97.7265) (width 0.254) (layer B.Cu) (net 9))
 (via (at 150.05 97.7265) (size 0.6) (layers F.Cu B.Cu) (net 9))
 (via (at 145.224 91.948) (size 0.6) (layers F.Cu B.Cu) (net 9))
 (segment (start 155.702 93.725) (end 163.828 93.725) (width 0.254) (layer F.Cu) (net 8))
 (segment (start 155.701 93.725) (end 155.702 93.725) (width 0.254) (layer F.Cu) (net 8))
 (segment (start 144.145 97.79) (end 145.669 96.266) (width 0.254) (layer F.Cu) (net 8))
 (segment (start 145.669 96.266) (end 145.669 93.7895) (width 0.254) (layer F.Cu) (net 8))
 (segment (start 145.669 93.7895) (end 146.748 92.71) (width 0.254) (layer F.Cu) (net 8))
 (segment (start 146.748 92.71) (end 154.686 92.71) (width 0.254) (layer F.Cu) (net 8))
 (segment (start 154.686 92.71) (end 155.701 93.725) (width 0.254) (layer F.Cu) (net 8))
 (segment (start 149.86 107.2) (end 149.86 106.299) (width 0.254) (layer F.Cu) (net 8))
 (segment (start 149.86 106.299) (end 150.241 105.918) (width 0.254) (layer F.Cu) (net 8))
 (segment (start 150.241 105.918) (end 152.019 104.14) (width 0.254) (layer B.Cu) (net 8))
 (segment (start 152.019 104.14) (end 152.019 97.409) (width 0.254) (layer B.Cu) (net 8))
 (segment (start 152.019 97.409) (end 155.702 93.726) (width 0.254) (layer B.Cu) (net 8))
 (segment (start 155.702 93.726) (end 155.702 93.725) (width 0.254) (layer F.Cu) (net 8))
 (segment (start 155.702 93.725) (end 155.701 93.725) (width 0.254) (layer F.Cu) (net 8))
 (via (at 150.241 105.918) (size 0.6) (layers F.Cu B.Cu) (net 8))
 (via (at 155.702 93.726) (size 0.6) (layers F.Cu B.Cu) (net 8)))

